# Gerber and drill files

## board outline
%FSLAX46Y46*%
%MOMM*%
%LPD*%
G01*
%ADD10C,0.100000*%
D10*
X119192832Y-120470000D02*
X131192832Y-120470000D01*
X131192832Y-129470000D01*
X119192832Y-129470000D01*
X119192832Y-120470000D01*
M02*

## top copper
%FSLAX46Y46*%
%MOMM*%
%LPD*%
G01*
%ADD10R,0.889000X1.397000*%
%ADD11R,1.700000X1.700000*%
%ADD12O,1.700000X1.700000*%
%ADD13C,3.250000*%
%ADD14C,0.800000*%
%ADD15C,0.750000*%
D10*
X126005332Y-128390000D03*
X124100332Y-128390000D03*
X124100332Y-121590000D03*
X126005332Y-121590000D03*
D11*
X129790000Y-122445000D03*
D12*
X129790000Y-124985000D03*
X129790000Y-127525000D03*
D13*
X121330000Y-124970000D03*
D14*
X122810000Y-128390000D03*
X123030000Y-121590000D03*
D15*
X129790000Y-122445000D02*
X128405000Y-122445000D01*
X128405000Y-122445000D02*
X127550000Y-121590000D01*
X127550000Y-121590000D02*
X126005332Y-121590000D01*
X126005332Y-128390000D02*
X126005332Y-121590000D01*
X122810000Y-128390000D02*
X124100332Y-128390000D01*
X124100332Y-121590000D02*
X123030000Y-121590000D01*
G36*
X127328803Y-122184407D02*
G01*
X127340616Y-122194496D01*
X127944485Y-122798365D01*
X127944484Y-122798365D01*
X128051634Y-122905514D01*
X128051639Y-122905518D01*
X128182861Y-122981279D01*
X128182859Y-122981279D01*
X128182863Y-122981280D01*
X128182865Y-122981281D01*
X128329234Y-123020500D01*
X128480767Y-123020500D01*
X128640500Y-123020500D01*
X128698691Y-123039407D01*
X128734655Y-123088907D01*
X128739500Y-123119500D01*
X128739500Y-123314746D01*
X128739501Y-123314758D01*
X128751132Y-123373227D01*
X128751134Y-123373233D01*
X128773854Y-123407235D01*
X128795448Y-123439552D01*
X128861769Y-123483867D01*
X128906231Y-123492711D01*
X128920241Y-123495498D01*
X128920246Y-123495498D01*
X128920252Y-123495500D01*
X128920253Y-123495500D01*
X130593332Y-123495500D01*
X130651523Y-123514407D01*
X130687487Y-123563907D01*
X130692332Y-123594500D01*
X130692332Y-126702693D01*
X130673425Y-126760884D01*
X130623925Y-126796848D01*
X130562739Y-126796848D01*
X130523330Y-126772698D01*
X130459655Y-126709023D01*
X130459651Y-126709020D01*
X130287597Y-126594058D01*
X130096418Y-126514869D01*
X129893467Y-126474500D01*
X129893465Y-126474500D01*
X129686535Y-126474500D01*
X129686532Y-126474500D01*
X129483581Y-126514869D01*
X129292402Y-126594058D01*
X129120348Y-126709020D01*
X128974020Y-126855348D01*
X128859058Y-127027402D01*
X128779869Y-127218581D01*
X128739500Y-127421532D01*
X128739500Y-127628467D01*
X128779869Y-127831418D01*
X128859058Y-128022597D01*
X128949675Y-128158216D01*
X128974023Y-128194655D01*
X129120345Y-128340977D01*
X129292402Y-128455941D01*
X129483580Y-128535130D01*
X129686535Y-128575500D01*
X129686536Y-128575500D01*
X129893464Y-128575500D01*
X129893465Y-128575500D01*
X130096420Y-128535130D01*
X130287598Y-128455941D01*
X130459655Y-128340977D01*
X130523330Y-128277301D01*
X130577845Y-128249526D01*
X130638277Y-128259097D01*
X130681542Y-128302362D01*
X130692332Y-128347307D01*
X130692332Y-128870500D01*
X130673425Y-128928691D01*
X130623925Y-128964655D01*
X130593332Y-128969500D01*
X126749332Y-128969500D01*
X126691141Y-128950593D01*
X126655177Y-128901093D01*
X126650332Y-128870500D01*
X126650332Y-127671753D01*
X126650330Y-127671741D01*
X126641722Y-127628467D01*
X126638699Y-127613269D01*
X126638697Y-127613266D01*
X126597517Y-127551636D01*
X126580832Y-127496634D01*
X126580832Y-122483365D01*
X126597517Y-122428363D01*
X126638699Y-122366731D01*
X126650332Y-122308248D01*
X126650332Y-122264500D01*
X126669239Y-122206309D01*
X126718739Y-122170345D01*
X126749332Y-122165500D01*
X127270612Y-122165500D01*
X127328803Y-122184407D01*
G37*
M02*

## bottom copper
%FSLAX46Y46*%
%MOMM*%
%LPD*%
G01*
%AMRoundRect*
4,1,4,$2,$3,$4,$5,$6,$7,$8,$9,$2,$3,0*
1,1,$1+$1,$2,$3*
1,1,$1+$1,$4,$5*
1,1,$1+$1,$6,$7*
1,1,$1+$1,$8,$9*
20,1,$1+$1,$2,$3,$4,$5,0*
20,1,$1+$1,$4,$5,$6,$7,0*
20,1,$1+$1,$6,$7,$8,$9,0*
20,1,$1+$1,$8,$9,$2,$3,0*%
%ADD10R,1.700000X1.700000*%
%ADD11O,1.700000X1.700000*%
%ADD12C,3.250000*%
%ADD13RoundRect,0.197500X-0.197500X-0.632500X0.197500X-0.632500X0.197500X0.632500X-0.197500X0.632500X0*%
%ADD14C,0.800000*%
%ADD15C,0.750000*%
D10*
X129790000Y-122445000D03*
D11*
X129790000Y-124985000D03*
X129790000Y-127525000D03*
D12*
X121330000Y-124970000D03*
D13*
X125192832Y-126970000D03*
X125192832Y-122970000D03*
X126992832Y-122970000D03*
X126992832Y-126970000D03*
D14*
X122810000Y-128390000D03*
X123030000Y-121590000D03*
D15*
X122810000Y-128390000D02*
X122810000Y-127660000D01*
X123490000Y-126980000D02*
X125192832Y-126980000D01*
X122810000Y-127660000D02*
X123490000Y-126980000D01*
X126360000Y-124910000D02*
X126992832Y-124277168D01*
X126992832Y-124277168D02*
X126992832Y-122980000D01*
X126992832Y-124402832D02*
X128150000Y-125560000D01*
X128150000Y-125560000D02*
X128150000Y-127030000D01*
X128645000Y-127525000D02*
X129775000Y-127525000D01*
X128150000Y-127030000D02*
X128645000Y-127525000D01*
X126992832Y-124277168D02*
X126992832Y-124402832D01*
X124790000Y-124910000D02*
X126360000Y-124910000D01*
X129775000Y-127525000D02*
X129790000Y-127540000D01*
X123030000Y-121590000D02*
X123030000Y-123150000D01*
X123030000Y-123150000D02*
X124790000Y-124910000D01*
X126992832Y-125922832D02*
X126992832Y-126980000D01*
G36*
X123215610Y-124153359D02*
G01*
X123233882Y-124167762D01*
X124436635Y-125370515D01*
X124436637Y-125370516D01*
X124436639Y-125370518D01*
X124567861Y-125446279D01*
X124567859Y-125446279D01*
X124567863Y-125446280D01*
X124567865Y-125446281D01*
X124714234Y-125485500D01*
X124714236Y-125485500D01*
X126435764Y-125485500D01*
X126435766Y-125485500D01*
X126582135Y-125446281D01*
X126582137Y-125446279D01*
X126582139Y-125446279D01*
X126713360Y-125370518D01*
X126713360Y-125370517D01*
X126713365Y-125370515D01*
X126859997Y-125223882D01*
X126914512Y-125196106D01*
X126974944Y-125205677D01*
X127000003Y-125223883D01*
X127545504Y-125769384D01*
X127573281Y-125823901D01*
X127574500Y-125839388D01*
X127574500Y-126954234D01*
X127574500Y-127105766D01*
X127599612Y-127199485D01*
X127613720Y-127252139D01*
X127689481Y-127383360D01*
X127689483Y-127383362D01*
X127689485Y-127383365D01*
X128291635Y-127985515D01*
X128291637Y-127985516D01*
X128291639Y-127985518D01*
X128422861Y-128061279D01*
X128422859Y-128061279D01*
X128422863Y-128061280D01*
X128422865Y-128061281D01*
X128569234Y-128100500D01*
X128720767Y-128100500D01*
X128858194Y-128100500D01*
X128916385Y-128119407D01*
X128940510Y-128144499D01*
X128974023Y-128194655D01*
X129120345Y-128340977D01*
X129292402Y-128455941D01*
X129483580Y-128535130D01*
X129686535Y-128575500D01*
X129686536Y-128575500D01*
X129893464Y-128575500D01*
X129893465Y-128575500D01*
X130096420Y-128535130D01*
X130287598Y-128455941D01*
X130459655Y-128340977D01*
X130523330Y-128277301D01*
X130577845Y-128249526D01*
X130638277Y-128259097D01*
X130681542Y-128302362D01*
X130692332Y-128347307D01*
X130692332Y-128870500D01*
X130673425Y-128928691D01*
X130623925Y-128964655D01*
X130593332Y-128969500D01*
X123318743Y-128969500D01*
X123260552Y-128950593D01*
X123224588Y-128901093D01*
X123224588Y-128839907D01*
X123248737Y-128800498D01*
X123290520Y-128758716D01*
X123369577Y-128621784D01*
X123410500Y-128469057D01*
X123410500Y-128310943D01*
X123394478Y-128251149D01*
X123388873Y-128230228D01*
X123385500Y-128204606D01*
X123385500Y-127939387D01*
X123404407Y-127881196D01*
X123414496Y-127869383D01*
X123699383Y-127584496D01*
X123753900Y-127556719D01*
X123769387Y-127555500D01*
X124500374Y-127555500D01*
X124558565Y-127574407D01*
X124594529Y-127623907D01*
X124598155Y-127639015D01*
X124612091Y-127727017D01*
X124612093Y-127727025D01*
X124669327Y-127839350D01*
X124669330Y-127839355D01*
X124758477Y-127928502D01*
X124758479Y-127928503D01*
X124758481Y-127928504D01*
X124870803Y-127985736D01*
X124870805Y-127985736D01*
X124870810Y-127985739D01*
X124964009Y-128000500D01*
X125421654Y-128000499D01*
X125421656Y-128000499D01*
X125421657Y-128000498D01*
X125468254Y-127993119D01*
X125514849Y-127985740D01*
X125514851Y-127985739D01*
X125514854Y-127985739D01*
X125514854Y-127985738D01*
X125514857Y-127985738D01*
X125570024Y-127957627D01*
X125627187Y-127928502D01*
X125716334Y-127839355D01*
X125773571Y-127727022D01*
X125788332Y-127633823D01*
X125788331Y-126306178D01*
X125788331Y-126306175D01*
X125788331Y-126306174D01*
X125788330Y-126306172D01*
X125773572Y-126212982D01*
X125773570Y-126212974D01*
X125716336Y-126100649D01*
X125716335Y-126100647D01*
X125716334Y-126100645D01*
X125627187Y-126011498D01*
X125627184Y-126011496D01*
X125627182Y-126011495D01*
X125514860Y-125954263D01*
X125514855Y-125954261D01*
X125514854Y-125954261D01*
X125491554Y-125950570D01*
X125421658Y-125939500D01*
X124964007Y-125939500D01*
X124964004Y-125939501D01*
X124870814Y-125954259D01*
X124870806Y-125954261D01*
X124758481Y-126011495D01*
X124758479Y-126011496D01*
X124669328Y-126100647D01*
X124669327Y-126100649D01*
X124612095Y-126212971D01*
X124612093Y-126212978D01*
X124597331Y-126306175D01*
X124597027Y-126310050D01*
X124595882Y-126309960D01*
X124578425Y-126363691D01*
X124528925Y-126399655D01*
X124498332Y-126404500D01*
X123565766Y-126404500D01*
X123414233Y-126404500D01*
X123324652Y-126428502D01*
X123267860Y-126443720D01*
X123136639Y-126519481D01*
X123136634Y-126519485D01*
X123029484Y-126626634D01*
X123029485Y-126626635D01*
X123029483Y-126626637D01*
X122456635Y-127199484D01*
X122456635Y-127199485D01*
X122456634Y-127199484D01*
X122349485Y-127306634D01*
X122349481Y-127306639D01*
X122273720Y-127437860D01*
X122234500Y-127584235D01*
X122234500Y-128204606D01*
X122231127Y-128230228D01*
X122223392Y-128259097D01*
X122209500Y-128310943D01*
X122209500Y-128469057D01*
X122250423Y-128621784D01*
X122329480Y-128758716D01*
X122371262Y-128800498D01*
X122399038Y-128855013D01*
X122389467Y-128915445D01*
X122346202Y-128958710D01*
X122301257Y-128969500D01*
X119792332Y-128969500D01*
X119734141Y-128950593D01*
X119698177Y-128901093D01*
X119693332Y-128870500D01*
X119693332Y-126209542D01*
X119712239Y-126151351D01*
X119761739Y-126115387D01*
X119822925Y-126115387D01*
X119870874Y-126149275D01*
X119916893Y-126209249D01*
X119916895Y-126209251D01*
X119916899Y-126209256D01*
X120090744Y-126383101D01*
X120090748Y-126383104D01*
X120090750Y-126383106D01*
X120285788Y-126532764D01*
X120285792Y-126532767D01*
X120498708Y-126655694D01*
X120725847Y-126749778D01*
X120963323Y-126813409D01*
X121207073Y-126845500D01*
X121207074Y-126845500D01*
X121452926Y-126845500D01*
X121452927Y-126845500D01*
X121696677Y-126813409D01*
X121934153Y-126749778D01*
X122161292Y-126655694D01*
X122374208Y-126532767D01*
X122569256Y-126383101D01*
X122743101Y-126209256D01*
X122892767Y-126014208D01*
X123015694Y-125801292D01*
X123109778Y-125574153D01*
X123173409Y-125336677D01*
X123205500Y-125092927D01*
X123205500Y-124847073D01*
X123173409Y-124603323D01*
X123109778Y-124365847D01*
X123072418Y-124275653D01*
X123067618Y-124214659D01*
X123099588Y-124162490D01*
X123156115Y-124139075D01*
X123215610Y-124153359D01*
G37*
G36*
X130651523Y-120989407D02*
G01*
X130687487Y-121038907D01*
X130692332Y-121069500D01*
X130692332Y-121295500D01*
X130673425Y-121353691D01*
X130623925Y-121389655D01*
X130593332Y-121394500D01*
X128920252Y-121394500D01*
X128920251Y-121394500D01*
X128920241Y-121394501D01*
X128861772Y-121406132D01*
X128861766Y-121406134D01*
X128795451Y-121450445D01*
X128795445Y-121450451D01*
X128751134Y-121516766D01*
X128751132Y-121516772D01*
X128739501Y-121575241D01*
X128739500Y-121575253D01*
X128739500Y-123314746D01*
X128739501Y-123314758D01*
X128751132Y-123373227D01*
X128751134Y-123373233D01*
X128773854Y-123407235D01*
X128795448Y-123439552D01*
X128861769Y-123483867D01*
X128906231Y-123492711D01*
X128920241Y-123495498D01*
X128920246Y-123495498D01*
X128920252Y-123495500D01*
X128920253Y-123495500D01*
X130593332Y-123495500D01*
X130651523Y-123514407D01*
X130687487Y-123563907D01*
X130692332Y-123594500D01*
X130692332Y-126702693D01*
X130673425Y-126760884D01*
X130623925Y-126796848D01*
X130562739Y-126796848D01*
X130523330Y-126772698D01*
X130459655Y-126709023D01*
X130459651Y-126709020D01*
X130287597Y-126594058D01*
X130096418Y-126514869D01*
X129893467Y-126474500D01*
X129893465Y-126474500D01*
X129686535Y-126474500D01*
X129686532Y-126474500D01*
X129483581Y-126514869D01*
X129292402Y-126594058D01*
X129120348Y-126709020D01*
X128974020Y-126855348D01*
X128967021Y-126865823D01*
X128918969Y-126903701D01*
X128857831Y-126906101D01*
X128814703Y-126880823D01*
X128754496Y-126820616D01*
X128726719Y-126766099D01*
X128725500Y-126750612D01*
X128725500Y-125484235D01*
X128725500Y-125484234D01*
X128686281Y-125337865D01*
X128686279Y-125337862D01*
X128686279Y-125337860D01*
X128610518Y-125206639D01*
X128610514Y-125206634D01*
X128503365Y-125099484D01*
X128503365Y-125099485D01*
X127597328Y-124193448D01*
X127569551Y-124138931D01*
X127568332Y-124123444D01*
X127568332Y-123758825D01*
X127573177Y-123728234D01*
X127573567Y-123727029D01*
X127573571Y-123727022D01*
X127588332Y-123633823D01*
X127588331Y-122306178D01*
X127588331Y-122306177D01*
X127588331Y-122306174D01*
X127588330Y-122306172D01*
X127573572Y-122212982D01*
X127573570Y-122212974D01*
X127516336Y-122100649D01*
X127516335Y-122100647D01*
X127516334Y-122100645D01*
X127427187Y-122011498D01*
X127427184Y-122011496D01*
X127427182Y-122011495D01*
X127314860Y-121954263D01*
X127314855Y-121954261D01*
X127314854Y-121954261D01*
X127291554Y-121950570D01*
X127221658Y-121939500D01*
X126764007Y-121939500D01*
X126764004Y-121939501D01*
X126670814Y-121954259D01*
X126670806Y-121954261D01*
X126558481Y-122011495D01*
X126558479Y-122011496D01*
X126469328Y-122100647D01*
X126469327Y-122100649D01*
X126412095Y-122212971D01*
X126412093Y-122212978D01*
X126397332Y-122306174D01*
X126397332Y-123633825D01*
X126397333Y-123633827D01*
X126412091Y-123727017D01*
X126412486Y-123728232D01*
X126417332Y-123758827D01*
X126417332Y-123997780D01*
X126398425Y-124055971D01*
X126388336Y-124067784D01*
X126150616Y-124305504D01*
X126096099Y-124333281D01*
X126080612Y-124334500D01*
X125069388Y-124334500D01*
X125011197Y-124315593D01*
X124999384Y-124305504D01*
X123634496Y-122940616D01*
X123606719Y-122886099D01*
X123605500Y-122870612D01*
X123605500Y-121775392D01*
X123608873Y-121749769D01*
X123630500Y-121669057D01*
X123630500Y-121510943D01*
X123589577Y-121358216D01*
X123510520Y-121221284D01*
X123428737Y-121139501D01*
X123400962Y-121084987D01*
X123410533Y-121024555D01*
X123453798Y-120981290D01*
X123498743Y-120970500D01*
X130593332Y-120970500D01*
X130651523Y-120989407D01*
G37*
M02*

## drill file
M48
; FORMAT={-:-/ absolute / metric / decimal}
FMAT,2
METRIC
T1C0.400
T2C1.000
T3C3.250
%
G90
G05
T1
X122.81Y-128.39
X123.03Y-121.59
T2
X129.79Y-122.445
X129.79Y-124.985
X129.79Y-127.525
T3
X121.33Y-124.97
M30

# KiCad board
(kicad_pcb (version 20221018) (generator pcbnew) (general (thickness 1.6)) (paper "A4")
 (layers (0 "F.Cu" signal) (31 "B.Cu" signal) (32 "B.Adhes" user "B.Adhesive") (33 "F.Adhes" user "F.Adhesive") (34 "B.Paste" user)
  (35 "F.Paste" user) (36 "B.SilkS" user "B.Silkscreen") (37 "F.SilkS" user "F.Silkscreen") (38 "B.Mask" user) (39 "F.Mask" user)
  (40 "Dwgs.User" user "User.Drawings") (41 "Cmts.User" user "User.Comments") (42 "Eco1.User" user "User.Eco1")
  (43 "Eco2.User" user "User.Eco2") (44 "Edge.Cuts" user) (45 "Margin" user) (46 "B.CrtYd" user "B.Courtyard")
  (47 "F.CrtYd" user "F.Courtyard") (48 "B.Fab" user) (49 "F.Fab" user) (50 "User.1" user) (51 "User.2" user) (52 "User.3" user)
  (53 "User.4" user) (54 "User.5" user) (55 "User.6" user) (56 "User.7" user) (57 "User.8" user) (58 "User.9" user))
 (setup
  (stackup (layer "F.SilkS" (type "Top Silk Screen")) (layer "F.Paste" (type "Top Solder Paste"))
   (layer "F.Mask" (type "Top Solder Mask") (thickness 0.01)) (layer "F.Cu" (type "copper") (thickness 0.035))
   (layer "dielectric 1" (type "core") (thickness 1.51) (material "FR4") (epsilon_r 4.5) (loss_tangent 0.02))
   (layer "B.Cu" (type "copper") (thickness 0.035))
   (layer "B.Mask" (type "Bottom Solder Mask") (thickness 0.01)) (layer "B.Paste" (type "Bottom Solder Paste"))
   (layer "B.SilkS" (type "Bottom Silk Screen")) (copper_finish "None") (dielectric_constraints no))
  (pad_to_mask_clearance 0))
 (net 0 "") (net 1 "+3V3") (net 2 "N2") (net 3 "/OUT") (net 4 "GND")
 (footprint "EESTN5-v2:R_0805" (layer "F.Cu") (at 125.052832 128.39 180)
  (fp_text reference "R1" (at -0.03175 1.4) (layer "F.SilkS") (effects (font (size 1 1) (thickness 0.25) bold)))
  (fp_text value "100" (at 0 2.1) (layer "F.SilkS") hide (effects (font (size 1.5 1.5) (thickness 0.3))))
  (pad "1" smd rect (at -0.9525 0 180) (size 0.889 1.397) (layers "F.Cu" "F.Paste" "F.Mask") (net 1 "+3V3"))
  (pad "2" smd rect (at 0.9525 0 180) (size 0.889 1.397) (layers "F.Cu" "F.Paste" "F.Mask") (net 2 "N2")))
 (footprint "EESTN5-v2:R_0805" (layer "F.Cu") (at 125.052832 121.59)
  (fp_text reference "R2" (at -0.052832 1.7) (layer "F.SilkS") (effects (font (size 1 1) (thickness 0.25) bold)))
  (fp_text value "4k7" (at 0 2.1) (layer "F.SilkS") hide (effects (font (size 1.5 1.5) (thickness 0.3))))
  (pad "1" smd rect (at -0.9525 0) (size 0.889 1.397) (layers "F.Cu" "F.Paste" "F.Mask") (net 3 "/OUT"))
  (pad "2" smd rect (at 0.9525 0) (size 0.889 1.397) (layers "F.Cu" "F.Paste" "F.Mask") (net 1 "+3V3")))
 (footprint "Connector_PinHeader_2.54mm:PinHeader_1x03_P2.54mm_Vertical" (layer "F.Cu") (at 129.79 122.445)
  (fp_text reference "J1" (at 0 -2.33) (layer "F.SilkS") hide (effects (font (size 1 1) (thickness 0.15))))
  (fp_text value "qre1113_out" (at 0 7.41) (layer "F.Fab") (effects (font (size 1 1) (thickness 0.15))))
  (pad "1" thru_hole rect (at 0 0) (size 1.7 1.7) (drill 1) (layers "*.Cu" "*.Mask") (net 1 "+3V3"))
  (pad "2" thru_hole oval (at 0 2.54) (size 1.7 1.7) (drill 1) (layers "*.Cu" "*.Mask") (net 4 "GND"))
  (pad "3" thru_hole oval (at 0 5.08) (size 1.7 1.7) (drill 1) (layers "*.Cu" "*.Mask") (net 3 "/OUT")))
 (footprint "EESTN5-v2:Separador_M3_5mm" (layer "F.Cu") (at 121.33 124.97 180)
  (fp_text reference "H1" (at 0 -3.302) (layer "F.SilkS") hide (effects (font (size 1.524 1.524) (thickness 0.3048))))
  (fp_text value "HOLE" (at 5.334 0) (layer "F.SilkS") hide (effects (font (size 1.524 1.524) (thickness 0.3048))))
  (pad "1" thru_hole circle (at 0 0 180) (size 3.25 3.25) (drill 3.25) (layers "*.Cu" "*.Mask")))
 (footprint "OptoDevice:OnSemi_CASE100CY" (layer "B.Cu") (at 126.092832 124.97)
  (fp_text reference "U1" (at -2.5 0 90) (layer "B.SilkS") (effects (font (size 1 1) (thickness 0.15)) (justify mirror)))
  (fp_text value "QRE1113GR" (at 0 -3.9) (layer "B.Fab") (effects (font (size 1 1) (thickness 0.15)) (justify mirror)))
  (pad "1" smd roundrect (at -0.9 2) (size 0.79 1.66) (layers "B.Cu" "B.Paste" "B.Mask") (roundrect_rratio 0.25) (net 2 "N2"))
  (pad "2" smd roundrect (at -0.9 -2) (size 0.79 1.66) (layers "B.Cu" "B.Paste" "B.Mask") (roundrect_rratio 0.25) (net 4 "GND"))
  (pad "3" smd roundrect (at 0.9 -2) (size 0.79 1.66) (layers "B.Cu" "B.Paste" "B.Mask") (roundrect_rratio 0.25) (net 3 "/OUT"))
  (pad "4" smd roundrect (at 0.9 2) (size 0.79 1.66) (layers "B.Cu" "B.Paste" "B.Mask") (roundrect_rratio 0.25) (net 4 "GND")))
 (gr_rect (start 119.192832 120.47) (end 131.192832 129.47) (stroke (width 0.1) (type default)) (fill none) (layer "Edge.Cuts"))
 (segment (start 129.79 122.445) (end 128.405 122.445) (width 0.75) (layer "F.Cu") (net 1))
 (segment (start 128.405 122.445) (end 127.55 121.59) (width 0.75) (layer "F.Cu") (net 1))
 (segment (start 127.55 121.59) (end 126.005332 121.59) (width 0.75) (layer "F.Cu") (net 1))
 (segment (start 126.005332 128.39) (end 126.005332 121.59) (width 0.75) (layer "F.Cu") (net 1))
 (segment (start 122.81 128.39) (end 124.100332 128.39) (width 0.75) (layer "F.Cu") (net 2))
 (via (at 122.81 128.39) (size 0.8) (drill 0.4) (layers "F.Cu" "B.Cu") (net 2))
 (segment (start 122.81 128.39) (end 122.81 127.66) (width 0.75) (layer "B.Cu") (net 2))
 (segment (start 123.49 126.98) (end 125.192832 126.98) (width 0.75) (layer "B.Cu") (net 2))
 (segment (start 122.81 127.66) (end 123.49 126.98) (width 0.75) (layer "B.Cu") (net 2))
 (segment (start 124.100332 121.59) (end 123.03 121.59) (width 0.75) (layer "F.Cu") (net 3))
 (via (at 123.03 121.59) (size 0.8) (drill 0.4) (layers "F.Cu" "B.Cu") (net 3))
 (segment (start 126.36 124.91) (end 126.992832 124.277168) (width 0.75) (layer "B.Cu") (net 3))
 (segment (start 126.992832 124.277168) (end 126.992832 122.98) (width 0.75) (layer "B.Cu") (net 3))
 (segment (start 126.992832 124.402832) (end 128.15 125.56) (width 0.75) (layer "B.Cu") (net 3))
 (segment (start 128.15 125.56) (end 128.15 127.03) (width 0.75) (layer "B.Cu") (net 3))
 (segment (start 128.645 127.525) (end 129.775 127.525) (width 0.75) (layer "B.Cu") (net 3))
 (segment (start 128.15 127.03) (end 128.645 127.525) (width 0.75) (layer "B.Cu") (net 3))
 (segment (start 126.992832 124.277168) (end 126.992832 124.402832) (width 0.75) (layer "B.Cu") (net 3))
 (segment (start 124.79 124.91) (end 126.36 124.91) (width 0.75) (layer "B.Cu") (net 3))
 (segment (start 129.775 127.525) (end 129.79 127.54) (width 0.75) (layer "B.Cu") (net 3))
 (segment (start 123.03 121.59) (end 123.03 123.15) (width 0.75) (layer "B.Cu") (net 3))
 (segment (start 123.03 123.15) (end 124.79 124.91) (width 0.75) (layer "B.Cu") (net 3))
 (segment (start 126.992832 125.922832) (end 126.992832 126.98) (width 0.75) (layer "B.Cu") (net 4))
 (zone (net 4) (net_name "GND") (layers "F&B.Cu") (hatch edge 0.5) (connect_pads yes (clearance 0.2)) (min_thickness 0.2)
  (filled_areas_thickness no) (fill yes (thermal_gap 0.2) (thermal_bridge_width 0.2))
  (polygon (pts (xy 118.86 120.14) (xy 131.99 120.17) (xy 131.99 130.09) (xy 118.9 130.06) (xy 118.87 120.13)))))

